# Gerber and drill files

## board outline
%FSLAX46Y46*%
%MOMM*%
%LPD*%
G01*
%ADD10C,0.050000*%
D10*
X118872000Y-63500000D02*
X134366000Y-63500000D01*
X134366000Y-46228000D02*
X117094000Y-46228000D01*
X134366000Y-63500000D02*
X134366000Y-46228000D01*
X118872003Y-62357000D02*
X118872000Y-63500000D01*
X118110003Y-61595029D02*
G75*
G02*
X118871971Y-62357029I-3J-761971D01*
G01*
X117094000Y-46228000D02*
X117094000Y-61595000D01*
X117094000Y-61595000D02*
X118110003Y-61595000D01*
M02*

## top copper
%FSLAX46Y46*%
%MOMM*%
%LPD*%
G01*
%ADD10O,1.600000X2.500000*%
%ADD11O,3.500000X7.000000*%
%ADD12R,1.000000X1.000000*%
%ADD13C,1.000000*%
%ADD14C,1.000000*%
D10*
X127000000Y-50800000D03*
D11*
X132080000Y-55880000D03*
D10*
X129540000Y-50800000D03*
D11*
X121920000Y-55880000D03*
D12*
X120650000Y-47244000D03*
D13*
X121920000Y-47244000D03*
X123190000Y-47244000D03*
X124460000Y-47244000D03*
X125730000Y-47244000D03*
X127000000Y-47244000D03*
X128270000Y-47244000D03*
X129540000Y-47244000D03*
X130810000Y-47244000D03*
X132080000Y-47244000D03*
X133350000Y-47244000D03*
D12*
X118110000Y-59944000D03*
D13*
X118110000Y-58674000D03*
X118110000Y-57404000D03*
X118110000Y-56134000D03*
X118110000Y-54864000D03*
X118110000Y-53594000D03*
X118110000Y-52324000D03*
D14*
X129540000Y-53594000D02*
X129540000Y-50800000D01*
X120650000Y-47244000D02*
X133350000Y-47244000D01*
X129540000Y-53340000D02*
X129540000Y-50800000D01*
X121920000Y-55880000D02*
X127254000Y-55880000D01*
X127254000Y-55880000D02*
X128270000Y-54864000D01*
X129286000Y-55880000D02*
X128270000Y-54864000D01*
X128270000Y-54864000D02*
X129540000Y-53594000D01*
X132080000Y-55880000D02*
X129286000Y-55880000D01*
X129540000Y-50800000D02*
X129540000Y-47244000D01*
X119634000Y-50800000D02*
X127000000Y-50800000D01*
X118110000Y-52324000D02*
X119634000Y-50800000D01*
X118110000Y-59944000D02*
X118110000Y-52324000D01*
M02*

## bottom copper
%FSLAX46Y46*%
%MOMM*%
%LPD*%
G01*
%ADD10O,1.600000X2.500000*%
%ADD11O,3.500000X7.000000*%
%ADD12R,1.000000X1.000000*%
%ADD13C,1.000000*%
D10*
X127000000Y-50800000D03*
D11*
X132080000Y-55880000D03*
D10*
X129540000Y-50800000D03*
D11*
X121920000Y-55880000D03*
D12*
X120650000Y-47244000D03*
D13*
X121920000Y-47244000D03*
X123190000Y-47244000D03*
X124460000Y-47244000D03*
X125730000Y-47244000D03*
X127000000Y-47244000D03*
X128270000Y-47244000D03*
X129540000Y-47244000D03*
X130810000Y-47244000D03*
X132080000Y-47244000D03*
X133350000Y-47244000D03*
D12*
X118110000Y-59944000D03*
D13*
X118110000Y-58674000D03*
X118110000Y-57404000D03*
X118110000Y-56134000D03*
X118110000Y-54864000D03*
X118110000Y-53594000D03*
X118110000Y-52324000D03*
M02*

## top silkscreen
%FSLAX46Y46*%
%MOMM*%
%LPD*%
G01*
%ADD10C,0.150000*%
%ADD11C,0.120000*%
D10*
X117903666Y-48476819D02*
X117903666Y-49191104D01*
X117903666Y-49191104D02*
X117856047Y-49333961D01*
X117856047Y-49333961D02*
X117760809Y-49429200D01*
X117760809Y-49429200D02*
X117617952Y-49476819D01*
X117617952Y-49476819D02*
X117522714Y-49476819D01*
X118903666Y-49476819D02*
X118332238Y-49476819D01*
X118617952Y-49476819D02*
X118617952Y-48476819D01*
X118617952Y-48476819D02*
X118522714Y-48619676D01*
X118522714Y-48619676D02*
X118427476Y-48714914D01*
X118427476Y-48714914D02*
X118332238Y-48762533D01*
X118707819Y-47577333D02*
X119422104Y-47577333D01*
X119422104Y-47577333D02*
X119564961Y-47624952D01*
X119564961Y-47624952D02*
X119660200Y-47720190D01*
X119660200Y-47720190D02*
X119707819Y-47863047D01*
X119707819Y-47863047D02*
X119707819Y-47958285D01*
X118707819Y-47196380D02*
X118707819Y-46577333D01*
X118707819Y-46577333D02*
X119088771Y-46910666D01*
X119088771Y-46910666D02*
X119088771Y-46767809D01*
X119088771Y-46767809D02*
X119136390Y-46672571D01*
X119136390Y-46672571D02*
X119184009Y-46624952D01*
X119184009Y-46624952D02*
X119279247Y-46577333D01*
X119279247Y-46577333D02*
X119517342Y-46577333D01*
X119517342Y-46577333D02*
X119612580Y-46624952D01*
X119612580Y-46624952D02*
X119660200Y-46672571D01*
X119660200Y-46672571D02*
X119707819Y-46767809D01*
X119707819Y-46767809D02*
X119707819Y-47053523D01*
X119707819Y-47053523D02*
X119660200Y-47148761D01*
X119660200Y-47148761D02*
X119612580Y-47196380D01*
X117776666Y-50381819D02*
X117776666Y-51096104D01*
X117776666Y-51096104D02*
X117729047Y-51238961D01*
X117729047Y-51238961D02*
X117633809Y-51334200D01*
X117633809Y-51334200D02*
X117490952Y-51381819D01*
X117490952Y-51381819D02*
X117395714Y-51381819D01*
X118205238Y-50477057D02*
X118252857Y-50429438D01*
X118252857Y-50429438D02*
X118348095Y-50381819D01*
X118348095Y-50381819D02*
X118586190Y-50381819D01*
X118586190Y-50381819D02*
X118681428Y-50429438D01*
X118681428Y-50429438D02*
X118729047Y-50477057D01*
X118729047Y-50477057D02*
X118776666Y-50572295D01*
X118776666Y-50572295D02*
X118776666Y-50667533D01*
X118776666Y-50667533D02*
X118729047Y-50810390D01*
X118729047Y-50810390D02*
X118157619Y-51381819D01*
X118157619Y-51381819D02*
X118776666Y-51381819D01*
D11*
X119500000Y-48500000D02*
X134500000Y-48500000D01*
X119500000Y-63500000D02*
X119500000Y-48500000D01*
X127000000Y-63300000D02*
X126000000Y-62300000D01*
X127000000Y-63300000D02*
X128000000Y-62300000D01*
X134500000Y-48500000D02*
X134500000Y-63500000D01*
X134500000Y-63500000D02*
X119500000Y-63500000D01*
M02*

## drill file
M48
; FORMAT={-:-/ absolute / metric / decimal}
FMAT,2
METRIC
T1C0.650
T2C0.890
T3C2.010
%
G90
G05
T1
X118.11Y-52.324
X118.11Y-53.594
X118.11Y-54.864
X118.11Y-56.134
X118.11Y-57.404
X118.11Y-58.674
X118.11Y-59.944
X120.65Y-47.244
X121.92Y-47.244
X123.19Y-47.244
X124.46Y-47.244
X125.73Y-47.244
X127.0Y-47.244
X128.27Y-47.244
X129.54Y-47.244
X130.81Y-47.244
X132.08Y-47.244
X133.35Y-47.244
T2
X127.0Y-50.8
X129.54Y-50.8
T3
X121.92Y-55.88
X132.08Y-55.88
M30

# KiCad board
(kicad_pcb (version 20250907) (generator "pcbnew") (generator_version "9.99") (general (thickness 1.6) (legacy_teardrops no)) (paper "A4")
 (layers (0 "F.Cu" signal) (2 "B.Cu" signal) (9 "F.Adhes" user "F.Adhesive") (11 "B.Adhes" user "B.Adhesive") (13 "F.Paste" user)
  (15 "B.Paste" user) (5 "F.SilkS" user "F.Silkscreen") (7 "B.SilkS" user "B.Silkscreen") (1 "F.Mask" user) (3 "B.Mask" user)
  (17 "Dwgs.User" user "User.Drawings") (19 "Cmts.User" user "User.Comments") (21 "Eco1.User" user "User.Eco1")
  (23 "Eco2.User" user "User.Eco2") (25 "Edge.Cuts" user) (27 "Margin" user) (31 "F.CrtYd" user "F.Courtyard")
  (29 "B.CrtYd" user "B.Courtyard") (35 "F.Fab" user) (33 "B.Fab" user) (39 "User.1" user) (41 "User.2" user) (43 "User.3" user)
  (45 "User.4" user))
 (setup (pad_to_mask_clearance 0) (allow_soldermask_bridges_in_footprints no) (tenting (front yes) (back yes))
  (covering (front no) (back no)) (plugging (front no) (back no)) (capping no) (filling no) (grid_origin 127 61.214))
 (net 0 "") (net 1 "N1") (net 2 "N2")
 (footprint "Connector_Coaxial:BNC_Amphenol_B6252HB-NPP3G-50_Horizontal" (layer "F.Cu") (at 127 50.8 180)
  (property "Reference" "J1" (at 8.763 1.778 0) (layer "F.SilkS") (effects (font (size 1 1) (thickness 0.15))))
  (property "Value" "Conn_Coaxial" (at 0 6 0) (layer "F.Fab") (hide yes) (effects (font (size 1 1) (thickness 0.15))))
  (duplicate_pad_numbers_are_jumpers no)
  (fp_line (start 7.5 2.3) (end -7.5 2.3) (stroke (width 0.12) (type solid)) (layer "F.SilkS"))
  (fp_line (start 7.5 -12.7) (end 7.5 2.3) (stroke (width 0.12) (type solid)) (layer "F.SilkS"))
  (fp_line (start 0 -12.5) (end 1 -11.5) (stroke (width 0.12) (type solid)) (layer "F.SilkS"))
  (fp_line (start 0 -12.5) (end -1 -11.5) (stroke (width 0.12) (type solid)) (layer "F.SilkS"))
  (fp_line (start -7.5 2.3) (end -7.5 -12.7) (stroke (width 0.12) (type solid)) (layer "F.SilkS"))
  (fp_line (start -7.5 -12.7) (end 7.5 -12.7) (stroke (width 0.12) (type solid)) (layer "F.SilkS"))
  (pad "1" thru_hole oval (at 0 0 180) (size 1.6 2.5) (drill 0.89) (layers "*.Cu" "*.Mask") (remove_unused_layers no) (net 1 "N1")
   (tenting (front none) (back none)))
  (pad "2" thru_hole oval (at -5.08 -5.08 180) (size 3.5 7) (drill 2.01) (layers "*.Cu" "*.Mask") (remove_unused_layers no) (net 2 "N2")
   (tenting (front none) (back none)))
  (pad "2" thru_hole oval (at -2.54 0 180) (size 1.6 2.5) (drill 0.89) (layers "*.Cu" "*.Mask") (remove_unused_layers no) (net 2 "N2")
   (tenting (front none) (back none)))
  (pad "2" thru_hole oval (at 5.08 -5.08 180) (size 3.5 7) (drill 2.01) (layers "*.Cu" "*.Mask") (remove_unused_layers no) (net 2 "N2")
   (tenting (front none) (back none))))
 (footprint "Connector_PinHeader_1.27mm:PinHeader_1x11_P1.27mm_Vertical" (layer "B.Cu") (at 120.65 47.244 -90)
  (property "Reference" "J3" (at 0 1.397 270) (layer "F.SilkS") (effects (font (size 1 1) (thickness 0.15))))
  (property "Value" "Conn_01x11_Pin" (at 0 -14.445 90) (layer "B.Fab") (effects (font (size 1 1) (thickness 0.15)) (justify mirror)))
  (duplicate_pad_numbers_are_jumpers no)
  (pad "1" thru_hole rect (at 0 0 270) (size 1 1) (drill 0.65) (layers "*.Cu" "*.Mask") (remove_unused_layers no) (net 2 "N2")
   (tenting (front none) (back none)))
  (pad "2" thru_hole circle (at 0 -1.27 270) (size 1 1) (drill 0.65) (layers "*.Cu" "*.Mask") (remove_unused_layers no) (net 2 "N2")
   (tenting (front none) (back none)))
  (pad "3" thru_hole circle (at 0 -2.54 270) (size 1 1) (drill 0.65) (layers "*.Cu" "*.Mask") (remove_unused_layers no) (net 2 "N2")
   (tenting (front none) (back none)))
  (pad "4" thru_hole circle (at 0 -3.81 270) (size 1 1) (drill 0.65) (layers "*.Cu" "*.Mask") (remove_unused_layers no) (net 2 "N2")
   (tenting (front none) (back none)))
  (pad "5" thru_hole circle (at 0 -5.08 270) (size 1 1) (drill 0.65) (layers "*.Cu" "*.Mask") (remove_unused_layers no) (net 2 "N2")
   (tenting (front none) (back none)))
  (pad "6" thru_hole circle (at 0 -6.35 270) (size 1 1) (drill 0.65) (layers "*.Cu" "*.Mask") (remove_unused_layers no) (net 2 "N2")
   (tenting (front none) (back none)))
  (pad "7" thru_hole circle (at 0 -7.62 270) (size 1 1) (drill 0.65) (layers "*.Cu" "*.Mask") (remove_unused_layers no) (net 2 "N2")
   (tenting (front none) (back none)))
  (pad "8" thru_hole circle (at 0 -8.89 270) (size 1 1) (drill 0.65) (layers "*.Cu" "*.Mask") (remove_unused_layers no) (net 2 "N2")
   (tenting (front none) (back none)))
  (pad "9" thru_hole circle (at 0 -10.16 270) (size 1 1) (drill 0.65) (layers "*.Cu" "*.Mask") (remove_unused_layers no) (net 2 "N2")
   (tenting (front none) (back none)))
  (pad "10" thru_hole circle (at 0 -11.43 270) (size 1 1) (drill 0.65) (layers "*.Cu" "*.Mask") (remove_unused_layers no) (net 2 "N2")
   (tenting (front none) (back none)))
  (pad "11" thru_hole circle (at 0 -12.7 270) (size 1 1) (drill 0.65) (layers "*.Cu" "*.Mask") (remove_unused_layers no) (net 2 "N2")
   (tenting (front none) (back none))))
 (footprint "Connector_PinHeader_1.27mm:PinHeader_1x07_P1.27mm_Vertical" (layer "B.Cu") (at 118.11 59.944)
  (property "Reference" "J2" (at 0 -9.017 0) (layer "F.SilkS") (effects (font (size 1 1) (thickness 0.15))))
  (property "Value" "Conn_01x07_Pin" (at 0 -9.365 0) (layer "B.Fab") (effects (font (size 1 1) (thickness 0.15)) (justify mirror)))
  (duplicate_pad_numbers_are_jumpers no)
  (pad "1" thru_hole rect (at 0 0) (size 1 1) (drill 0.65) (layers "*.Cu" "*.Mask") (remove_unused_layers no) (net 1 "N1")
   (tenting (front none) (back none)))
  (pad "2" thru_hole circle (at 0 -1.27) (size 1 1) (drill 0.65) (layers "*.Cu" "*.Mask") (remove_unused_layers no) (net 1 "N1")
   (tenting (front none) (back none)))
  (pad "3" thru_hole circle (at 0 -2.54) (size 1 1) (drill 0.65) (layers "*.Cu" "*.Mask") (remove_unused_layers no) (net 1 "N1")
   (tenting (front none) (back none)))
  (pad "4" thru_hole circle (at 0 -3.81) (size 1 1) (drill 0.65) (layers "*.Cu" "*.Mask") (remove_unused_layers no) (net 1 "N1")
   (tenting (front none) (back none)))
  (pad "5" thru_hole circle (at 0 -5.08) (size 1 1) (drill 0.65) (layers "*.Cu" "*.Mask") (remove_unused_layers no) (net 1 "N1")
   (tenting (front none) (back none)))
  (pad "6" thru_hole circle (at 0 -6.35) (size 1 1) (drill 0.65) (layers "*.Cu" "*.Mask") (remove_unused_layers no) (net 1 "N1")
   (tenting (front none) (back none)))
  (pad "7" thru_hole circle (at 0 -7.62) (size 1 1) (drill 0.65) (layers "*.Cu" "*.Mask") (remove_unused_layers no) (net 1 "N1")
   (tenting (front none) (back none))))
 (gr_line (start 118.872 63.5) (end 134.366 63.5) (stroke (width 0.05) (type default)) (layer "Edge.Cuts"))
 (gr_line (start 134.366 46.228) (end 117.094 46.228) (stroke (width 0.05) (type default)) (layer "Edge.Cuts"))
 (gr_line (start 134.366 63.5) (end 134.366 46.228) (stroke (width 0.05) (type default)) (layer "Edge.Cuts"))
 (gr_line (start 118.872003 62.357) (end 118.872 63.5) (stroke (width 0.05) (type default)) (layer "Edge.Cuts"))
 (gr_arc (start 118.110003 61.595029) (mid 118.648818 61.818214) (end 118.872003 62.357029) (stroke (width 0.05) (type default))
  (layer "Edge.Cuts"))
 (gr_line (start 117.094 46.228) (end 117.094 61.595) (stroke (width 0.05) (type default)) (layer "Edge.Cuts"))
 (gr_line (start 117.094 61.595) (end 118.110003 61.595) (stroke (width 0.05) (type default)) (layer "Edge.Cuts"))
 (segment (start 129.54 53.594) (end 129.54 50.8) (width 1) (layer "F.Cu") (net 2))
 (segment (start 120.65 47.244) (end 133.35 47.244) (width 1) (layer "F.Cu") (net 2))
 (segment (start 129.54 53.34) (end 129.54 50.8) (width 1) (layer "F.Cu") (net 2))
 (segment (start 121.92 55.88) (end 127.254 55.88) (width 1) (layer "F.Cu") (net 2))
 (segment (start 127.254 55.88) (end 128.27 54.864) (width 1) (layer "F.Cu") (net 2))
 (segment (start 129.286 55.88) (end 128.27 54.864) (width 1) (layer "F.Cu") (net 2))
 (segment (start 128.27 54.864) (end 129.54 53.594) (width 1) (layer "F.Cu") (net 2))
 (segment (start 132.08 55.88) (end 129.286 55.88) (width 1) (layer "F.Cu") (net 2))
 (segment (start 129.54 50.8) (end 129.54 47.244) (width 1) (layer "F.Cu") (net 2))
 (segment (start 119.634 50.8) (end 127 50.8) (width 1) (layer "F.Cu") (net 1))
 (segment (start 118.11 52.324) (end 119.634 50.8) (width 1) (layer "F.Cu") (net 1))
 (segment (start 118.11 59.944) (end 118.11 52.324) (width 1) (layer "F.Cu") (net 1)))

